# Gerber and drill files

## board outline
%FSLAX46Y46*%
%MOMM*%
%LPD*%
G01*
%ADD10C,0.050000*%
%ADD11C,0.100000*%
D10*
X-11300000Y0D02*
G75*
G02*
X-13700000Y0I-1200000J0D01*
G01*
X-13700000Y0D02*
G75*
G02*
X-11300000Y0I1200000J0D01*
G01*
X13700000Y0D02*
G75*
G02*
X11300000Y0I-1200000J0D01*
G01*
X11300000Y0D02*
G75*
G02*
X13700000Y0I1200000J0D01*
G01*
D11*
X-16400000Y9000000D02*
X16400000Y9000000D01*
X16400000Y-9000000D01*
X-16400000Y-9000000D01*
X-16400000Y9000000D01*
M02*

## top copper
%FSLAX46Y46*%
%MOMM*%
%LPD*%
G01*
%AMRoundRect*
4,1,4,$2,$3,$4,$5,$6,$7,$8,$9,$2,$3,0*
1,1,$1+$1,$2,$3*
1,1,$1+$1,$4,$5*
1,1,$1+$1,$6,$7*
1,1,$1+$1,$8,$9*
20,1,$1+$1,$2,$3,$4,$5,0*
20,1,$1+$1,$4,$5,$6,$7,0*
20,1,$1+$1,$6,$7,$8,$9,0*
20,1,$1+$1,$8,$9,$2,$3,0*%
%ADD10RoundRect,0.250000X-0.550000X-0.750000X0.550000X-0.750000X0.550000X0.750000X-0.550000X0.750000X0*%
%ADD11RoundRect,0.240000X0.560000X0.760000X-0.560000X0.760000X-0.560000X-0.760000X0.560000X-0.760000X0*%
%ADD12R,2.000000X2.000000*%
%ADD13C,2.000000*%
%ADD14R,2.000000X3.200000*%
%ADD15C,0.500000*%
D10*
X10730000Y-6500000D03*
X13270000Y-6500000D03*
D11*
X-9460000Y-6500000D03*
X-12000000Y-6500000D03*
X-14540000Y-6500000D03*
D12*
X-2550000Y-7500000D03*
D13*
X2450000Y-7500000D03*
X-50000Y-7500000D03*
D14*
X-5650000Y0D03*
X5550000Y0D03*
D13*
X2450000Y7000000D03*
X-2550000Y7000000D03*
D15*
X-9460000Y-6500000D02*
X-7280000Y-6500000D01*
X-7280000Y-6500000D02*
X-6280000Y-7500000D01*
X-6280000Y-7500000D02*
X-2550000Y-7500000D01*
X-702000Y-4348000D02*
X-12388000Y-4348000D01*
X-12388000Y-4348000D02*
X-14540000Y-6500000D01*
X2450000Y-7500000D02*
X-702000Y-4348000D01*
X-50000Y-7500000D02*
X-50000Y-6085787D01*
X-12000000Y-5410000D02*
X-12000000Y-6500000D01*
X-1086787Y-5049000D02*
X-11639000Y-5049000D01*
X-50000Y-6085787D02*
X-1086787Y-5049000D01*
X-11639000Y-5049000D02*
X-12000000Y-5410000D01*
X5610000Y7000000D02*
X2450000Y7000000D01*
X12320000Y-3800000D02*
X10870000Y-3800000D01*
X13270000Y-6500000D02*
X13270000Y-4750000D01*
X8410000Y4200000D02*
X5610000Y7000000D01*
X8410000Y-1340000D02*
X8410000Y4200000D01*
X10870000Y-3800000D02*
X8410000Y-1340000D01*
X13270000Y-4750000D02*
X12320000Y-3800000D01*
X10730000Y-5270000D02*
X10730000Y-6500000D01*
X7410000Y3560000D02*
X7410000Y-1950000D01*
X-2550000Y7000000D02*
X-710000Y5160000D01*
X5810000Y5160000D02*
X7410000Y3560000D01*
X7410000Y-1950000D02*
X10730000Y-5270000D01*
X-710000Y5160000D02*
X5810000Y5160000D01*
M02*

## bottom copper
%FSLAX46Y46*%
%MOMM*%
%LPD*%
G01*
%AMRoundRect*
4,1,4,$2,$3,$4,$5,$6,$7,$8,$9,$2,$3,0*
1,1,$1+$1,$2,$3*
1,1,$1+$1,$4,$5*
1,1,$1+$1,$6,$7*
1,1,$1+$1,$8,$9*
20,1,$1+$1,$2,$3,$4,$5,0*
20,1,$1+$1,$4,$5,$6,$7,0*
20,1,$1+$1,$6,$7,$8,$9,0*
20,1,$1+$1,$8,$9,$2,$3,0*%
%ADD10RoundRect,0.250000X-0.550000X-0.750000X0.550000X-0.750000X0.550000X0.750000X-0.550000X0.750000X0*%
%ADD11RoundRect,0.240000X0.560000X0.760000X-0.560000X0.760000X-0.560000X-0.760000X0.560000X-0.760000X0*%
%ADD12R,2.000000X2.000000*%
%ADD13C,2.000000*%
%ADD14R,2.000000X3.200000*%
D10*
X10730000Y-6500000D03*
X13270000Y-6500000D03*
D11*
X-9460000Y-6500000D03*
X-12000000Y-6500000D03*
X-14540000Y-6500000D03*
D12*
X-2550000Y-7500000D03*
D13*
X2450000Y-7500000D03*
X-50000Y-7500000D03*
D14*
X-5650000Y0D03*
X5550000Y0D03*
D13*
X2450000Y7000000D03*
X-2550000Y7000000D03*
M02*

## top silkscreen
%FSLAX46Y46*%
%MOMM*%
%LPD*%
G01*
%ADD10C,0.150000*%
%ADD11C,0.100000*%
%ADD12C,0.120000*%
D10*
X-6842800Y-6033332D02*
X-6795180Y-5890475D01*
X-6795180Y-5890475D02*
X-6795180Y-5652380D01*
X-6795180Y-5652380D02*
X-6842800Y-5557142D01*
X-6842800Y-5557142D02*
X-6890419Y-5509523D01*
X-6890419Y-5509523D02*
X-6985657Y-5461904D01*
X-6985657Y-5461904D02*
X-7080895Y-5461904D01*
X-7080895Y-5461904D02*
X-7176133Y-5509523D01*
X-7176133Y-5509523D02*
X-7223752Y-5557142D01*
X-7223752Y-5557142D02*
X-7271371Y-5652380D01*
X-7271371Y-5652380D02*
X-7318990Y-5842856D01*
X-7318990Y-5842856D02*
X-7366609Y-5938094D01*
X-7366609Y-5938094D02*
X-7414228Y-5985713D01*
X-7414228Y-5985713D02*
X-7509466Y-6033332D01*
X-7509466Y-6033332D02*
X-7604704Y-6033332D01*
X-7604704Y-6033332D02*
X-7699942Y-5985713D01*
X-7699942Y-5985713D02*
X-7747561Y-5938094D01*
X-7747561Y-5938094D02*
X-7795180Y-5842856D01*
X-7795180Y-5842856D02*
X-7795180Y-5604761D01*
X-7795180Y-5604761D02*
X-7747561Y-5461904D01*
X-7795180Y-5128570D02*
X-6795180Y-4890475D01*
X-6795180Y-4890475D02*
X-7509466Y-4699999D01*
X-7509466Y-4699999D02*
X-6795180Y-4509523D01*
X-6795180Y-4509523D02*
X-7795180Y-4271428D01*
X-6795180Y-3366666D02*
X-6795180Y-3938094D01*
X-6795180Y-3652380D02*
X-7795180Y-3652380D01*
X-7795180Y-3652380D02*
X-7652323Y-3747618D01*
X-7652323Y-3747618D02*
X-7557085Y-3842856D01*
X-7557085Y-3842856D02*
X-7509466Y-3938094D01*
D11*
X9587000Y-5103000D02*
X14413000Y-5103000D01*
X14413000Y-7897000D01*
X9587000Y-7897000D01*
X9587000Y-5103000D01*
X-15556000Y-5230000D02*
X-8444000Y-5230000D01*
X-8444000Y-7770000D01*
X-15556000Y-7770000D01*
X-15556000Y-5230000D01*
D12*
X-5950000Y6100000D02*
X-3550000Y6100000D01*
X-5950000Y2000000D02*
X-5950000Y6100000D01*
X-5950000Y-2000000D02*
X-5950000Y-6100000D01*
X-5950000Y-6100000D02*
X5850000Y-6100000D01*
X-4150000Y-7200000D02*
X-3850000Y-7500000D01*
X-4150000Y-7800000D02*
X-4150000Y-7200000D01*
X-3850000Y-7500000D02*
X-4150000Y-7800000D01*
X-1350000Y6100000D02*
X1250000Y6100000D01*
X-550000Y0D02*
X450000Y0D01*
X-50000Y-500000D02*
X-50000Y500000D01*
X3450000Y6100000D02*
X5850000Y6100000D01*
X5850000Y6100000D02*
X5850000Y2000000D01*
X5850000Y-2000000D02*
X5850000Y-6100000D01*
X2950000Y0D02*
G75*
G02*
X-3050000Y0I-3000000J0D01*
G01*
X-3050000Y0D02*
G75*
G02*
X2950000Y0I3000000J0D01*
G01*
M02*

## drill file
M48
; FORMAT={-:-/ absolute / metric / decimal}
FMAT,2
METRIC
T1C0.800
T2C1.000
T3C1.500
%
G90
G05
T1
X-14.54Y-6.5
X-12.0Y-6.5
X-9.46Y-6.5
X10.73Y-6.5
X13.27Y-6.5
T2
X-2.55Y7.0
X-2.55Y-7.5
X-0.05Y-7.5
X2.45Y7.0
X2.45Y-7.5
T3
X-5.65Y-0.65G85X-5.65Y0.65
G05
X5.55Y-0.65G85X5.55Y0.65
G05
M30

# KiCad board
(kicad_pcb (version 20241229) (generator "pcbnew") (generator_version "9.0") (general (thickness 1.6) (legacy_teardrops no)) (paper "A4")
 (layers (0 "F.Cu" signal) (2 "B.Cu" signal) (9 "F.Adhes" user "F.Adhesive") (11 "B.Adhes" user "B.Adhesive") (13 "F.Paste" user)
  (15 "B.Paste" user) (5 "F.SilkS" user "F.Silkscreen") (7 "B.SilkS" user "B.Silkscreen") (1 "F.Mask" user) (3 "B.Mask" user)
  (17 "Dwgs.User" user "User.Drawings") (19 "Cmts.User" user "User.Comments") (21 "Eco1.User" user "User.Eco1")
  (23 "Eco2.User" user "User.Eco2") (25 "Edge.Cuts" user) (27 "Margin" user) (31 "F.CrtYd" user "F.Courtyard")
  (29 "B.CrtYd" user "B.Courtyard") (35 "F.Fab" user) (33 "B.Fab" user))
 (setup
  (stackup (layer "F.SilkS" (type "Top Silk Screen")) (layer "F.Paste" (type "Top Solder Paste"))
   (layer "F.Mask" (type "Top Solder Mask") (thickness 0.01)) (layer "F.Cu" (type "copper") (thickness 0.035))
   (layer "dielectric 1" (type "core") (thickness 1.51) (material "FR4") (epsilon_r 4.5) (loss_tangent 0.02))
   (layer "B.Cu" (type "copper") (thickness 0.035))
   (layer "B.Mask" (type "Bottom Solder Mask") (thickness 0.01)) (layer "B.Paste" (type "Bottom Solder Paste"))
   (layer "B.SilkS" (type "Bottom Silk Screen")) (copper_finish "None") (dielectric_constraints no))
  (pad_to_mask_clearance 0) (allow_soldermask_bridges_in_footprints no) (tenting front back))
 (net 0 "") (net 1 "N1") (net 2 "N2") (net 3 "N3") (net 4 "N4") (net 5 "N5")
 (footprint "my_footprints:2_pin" (layer "F.Cu") (at 12 6.5)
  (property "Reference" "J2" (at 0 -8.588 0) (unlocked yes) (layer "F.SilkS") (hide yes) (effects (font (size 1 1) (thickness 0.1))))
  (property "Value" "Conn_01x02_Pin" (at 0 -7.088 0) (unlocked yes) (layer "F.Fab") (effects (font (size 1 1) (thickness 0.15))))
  (fp_rect (start -2.413 -1.397) (end 2.413 1.397) (stroke (width 0.1) (type default)) (fill no) (layer "F.SilkS"))
  (pad "1" thru_hole roundrect (at -1.27 0) (size 1.6 2) (drill 0.8) (layers "*.Cu" "*.Mask") (remove_unused_layers no)
   (roundrect_rratio 0.15625) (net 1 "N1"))
  (pad "2" thru_hole roundrect (at 1.27 0) (size 1.6 2) (drill 0.8) (layers "*.Cu" "*.Mask") (remove_unused_layers no)
   (roundrect_rratio 0.15625) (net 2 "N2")))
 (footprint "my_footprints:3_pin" (layer "F.Cu") (at -12 6.5 180)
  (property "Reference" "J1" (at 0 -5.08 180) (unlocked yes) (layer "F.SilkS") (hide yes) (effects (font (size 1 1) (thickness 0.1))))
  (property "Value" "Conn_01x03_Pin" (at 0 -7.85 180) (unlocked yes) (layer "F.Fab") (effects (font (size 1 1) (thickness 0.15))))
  (fp_rect (start -3.556 -1.27) (end 3.556 1.27) (stroke (width 0.1) (type default)) (fill no) (layer "F.SilkS"))
  (pad "1" thru_hole roundrect (at -2.54 0 180) (size 1.6 2) (drill 0.8) (layers "*.Cu" "*.Mask") (remove_unused_layers no)
   (roundrect_rratio 0.15) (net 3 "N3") (thermal_bridge_angle 45))
  (pad "2" thru_hole roundrect (at 0 0 180) (size 1.6 2) (drill 0.8) (layers "*.Cu" "*.Mask") (remove_unused_layers no)
   (roundrect_rratio 0.15) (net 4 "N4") (thermal_bridge_angle 45))
  (pad "3" thru_hole roundrect (at 2.54 0 180) (size 1.6 2) (drill 0.8) (layers "*.Cu" "*.Mask") (remove_unused_layers no)
   (roundrect_rratio 0.15) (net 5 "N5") (thermal_bridge_angle 45)))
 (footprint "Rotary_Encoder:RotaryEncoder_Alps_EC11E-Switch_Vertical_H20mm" (layer "F.Cu") (at -2.55 7.5 90)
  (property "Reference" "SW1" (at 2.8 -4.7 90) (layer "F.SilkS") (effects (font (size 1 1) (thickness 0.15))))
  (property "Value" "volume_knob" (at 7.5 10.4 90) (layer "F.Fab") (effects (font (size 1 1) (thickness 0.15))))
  (fp_line (start 13.6 -3.4) (end 13.6 -1) (stroke (width 0.12) (type solid)) (layer "F.SilkS"))
  (fp_line (start 9.5 -3.4) (end 13.6 -3.4) (stroke (width 0.12) (type solid)) (layer "F.SilkS"))
  (fp_line (start 5.5 -3.4) (end 1.4 -3.4) (stroke (width 0.12) (type solid)) (layer "F.SilkS"))
  (fp_line (start 1.4 -3.4) (end 1.4 8.4) (stroke (width 0.12) (type solid)) (layer "F.SilkS"))
  (fp_line (start 0.3 -1.6) (end 0 -1.3) (stroke (width 0.12) (type solid)) (layer "F.SilkS"))
  (fp_line (start -0.3 -1.6) (end 0.3 -1.6) (stroke (width 0.12) (type solid)) (layer "F.SilkS"))
  (fp_line (start 0 -1.3) (end -0.3 -1.6) (stroke (width 0.12) (type solid)) (layer "F.SilkS"))
  (fp_line (start 13.6 1.2) (end 13.6 3.8) (stroke (width 0.12) (type solid)) (layer "F.SilkS"))
  (fp_line (start 7.5 2) (end 7.5 3) (stroke (width 0.12) (type solid)) (layer "F.SilkS"))
  (fp_line (start 7 2.5) (end 8 2.5) (stroke (width 0.12) (type solid)) (layer "F.SilkS"))
  (fp_line (start 13.6 6) (end 13.6 8.4) (stroke (width 0.12) (type solid)) (layer "F.SilkS"))
  (fp_line (start 13.6 8.4) (end 9.5 8.4) (stroke (width 0.12) (type solid)) (layer "F.SilkS"))
  (fp_line (start 5.5 8.4) (end 1.4 8.4) (stroke (width 0.12) (type solid)) (layer "F.SilkS"))
  (fp_circle (center 7.5 2.5) (end 10.5 2.5) (stroke (width 0.12) (type solid)) (fill no) (layer "F.SilkS"))
  (pad "A" thru_hole rect (at 0 0 90) (size 2 2) (drill 1) (layers "*.Cu" "*.Mask") (remove_unused_layers no) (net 3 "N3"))
  (pad "B" thru_hole circle (at 0 5 90) (size 2 2) (drill 1) (layers "*.Cu" "*.Mask") (remove_unused_layers no) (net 5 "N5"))
  (pad "C" thru_hole circle (at 0 2.5 90) (size 2 2) (drill 1) (layers "*.Cu" "*.Mask") (remove_unused_layers no) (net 4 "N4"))
  (pad "MP" thru_hole rect (at 7.5 -3.1 90) (size 3.2 2) (drill oval 2.8 1.5) (layers "*.Cu" "*.Mask") (remove_unused_layers no))
  (pad "MP" thru_hole rect (at 7.5 8.1 90) (size 3.2 2) (drill oval 2.8 1.5) (layers "*.Cu" "*.Mask") (remove_unused_layers no))
  (pad "S1" thru_hole circle (at 14.5 5 90) (size 2 2) (drill 1) (layers "*.Cu" "*.Mask") (remove_unused_layers no) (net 2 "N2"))
  (pad "S2" thru_hole circle (at 14.5 0 90) (size 2 2) (drill 1) (layers "*.Cu" "*.Mask") (remove_unused_layers no) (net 1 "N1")))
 (gr_circle (center -12.5 0) (end -11.3 0) (stroke (width 0.05) (type solid)) (fill no) (layer "Edge.Cuts"))
 (gr_circle (center 12.5 0) (end 13.7 0) (stroke (width 0.05) (type solid)) (fill no) (layer "Edge.Cuts"))
 (gr_rect (start -16.4 -9) (end 16.4 9) (stroke (width 0.1) (type solid)) (fill no) (layer "Edge.Cuts"))
 (segment (start -9.46 6.5) (end -7.28 6.5) (width 0.5) (layer "F.Cu") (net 3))
 (segment (start -7.28 6.5) (end -6.28 7.5) (width 0.5) (layer "F.Cu") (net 3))
 (segment (start -6.28 7.5) (end -2.55 7.5) (width 0.5) (layer "F.Cu") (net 3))
 (segment (start -0.702 4.348) (end -12.388 4.348) (width 0.5) (layer "F.Cu") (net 5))
 (segment (start -12.388 4.348) (end -14.54 6.5) (width 0.5) (layer "F.Cu") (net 5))
 (segment (start 2.45 7.5) (end -0.702 4.348) (width 0.5) (layer "F.Cu") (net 5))
 (segment (start -0.05 7.5) (end -0.05 6.085787) (width 0.5) (layer "F.Cu") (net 4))
 (segment (start -12 5.41) (end -12 6.5) (width 0.5) (layer "F.Cu") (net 4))
 (segment (start -1.086787 5.049) (end -11.639 5.049) (width 0.5) (layer "F.Cu") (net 4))
 (segment (start -0.05 6.085787) (end -1.086787 5.049) (width 0.5) (layer "F.Cu") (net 4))
 (segment (start -11.639 5.049) (end -12 5.41) (width 0.5) (layer "F.Cu") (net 4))
 (segment (start 5.61 -7) (end 2.45 -7) (width 0.5) (layer "F.Cu") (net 2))
 (segment (start 12.32 3.8) (end 10.87 3.8) (width 0.5) (layer "F.Cu") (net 2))
 (segment (start 13.27 6.5) (end 13.27 4.75) (width 0.5) (layer "F.Cu") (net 2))
 (segment (start 8.41 -4.2) (end 5.61 -7) (width 0.5) (layer "F.Cu") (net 2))
 (segment (start 8.41 1.34) (end 8.41 -4.2) (width 0.5) (layer "F.Cu") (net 2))
 (segment (start 10.87 3.8) (end 8.41 1.34) (width 0.5) (layer "F.Cu") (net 2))
 (segment (start 13.27 4.75) (end 12.32 3.8) (width 0.5) (layer "F.Cu") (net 2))
 (segment (start 10.73 5.27) (end 10.73 6.5) (width 0.5) (layer "F.Cu") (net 1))
 (segment (start 7.41 -3.56) (end 7.41 1.95) (width 0.5) (layer "F.Cu") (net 1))
 (segment (start -2.55 -7) (end -0.71 -5.16) (width 0.5) (layer "F.Cu") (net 1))
 (segment (start 5.81 -5.16) (end 7.41 -3.56) (width 0.5) (layer "F.Cu") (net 1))
 (segment (start 7.41 1.95) (end 10.73 5.27) (width 0.5) (layer "F.Cu") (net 1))
 (segment (start -0.71 -5.16) (end 5.81 -5.16) (width 0.5) (layer "F.Cu") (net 1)))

